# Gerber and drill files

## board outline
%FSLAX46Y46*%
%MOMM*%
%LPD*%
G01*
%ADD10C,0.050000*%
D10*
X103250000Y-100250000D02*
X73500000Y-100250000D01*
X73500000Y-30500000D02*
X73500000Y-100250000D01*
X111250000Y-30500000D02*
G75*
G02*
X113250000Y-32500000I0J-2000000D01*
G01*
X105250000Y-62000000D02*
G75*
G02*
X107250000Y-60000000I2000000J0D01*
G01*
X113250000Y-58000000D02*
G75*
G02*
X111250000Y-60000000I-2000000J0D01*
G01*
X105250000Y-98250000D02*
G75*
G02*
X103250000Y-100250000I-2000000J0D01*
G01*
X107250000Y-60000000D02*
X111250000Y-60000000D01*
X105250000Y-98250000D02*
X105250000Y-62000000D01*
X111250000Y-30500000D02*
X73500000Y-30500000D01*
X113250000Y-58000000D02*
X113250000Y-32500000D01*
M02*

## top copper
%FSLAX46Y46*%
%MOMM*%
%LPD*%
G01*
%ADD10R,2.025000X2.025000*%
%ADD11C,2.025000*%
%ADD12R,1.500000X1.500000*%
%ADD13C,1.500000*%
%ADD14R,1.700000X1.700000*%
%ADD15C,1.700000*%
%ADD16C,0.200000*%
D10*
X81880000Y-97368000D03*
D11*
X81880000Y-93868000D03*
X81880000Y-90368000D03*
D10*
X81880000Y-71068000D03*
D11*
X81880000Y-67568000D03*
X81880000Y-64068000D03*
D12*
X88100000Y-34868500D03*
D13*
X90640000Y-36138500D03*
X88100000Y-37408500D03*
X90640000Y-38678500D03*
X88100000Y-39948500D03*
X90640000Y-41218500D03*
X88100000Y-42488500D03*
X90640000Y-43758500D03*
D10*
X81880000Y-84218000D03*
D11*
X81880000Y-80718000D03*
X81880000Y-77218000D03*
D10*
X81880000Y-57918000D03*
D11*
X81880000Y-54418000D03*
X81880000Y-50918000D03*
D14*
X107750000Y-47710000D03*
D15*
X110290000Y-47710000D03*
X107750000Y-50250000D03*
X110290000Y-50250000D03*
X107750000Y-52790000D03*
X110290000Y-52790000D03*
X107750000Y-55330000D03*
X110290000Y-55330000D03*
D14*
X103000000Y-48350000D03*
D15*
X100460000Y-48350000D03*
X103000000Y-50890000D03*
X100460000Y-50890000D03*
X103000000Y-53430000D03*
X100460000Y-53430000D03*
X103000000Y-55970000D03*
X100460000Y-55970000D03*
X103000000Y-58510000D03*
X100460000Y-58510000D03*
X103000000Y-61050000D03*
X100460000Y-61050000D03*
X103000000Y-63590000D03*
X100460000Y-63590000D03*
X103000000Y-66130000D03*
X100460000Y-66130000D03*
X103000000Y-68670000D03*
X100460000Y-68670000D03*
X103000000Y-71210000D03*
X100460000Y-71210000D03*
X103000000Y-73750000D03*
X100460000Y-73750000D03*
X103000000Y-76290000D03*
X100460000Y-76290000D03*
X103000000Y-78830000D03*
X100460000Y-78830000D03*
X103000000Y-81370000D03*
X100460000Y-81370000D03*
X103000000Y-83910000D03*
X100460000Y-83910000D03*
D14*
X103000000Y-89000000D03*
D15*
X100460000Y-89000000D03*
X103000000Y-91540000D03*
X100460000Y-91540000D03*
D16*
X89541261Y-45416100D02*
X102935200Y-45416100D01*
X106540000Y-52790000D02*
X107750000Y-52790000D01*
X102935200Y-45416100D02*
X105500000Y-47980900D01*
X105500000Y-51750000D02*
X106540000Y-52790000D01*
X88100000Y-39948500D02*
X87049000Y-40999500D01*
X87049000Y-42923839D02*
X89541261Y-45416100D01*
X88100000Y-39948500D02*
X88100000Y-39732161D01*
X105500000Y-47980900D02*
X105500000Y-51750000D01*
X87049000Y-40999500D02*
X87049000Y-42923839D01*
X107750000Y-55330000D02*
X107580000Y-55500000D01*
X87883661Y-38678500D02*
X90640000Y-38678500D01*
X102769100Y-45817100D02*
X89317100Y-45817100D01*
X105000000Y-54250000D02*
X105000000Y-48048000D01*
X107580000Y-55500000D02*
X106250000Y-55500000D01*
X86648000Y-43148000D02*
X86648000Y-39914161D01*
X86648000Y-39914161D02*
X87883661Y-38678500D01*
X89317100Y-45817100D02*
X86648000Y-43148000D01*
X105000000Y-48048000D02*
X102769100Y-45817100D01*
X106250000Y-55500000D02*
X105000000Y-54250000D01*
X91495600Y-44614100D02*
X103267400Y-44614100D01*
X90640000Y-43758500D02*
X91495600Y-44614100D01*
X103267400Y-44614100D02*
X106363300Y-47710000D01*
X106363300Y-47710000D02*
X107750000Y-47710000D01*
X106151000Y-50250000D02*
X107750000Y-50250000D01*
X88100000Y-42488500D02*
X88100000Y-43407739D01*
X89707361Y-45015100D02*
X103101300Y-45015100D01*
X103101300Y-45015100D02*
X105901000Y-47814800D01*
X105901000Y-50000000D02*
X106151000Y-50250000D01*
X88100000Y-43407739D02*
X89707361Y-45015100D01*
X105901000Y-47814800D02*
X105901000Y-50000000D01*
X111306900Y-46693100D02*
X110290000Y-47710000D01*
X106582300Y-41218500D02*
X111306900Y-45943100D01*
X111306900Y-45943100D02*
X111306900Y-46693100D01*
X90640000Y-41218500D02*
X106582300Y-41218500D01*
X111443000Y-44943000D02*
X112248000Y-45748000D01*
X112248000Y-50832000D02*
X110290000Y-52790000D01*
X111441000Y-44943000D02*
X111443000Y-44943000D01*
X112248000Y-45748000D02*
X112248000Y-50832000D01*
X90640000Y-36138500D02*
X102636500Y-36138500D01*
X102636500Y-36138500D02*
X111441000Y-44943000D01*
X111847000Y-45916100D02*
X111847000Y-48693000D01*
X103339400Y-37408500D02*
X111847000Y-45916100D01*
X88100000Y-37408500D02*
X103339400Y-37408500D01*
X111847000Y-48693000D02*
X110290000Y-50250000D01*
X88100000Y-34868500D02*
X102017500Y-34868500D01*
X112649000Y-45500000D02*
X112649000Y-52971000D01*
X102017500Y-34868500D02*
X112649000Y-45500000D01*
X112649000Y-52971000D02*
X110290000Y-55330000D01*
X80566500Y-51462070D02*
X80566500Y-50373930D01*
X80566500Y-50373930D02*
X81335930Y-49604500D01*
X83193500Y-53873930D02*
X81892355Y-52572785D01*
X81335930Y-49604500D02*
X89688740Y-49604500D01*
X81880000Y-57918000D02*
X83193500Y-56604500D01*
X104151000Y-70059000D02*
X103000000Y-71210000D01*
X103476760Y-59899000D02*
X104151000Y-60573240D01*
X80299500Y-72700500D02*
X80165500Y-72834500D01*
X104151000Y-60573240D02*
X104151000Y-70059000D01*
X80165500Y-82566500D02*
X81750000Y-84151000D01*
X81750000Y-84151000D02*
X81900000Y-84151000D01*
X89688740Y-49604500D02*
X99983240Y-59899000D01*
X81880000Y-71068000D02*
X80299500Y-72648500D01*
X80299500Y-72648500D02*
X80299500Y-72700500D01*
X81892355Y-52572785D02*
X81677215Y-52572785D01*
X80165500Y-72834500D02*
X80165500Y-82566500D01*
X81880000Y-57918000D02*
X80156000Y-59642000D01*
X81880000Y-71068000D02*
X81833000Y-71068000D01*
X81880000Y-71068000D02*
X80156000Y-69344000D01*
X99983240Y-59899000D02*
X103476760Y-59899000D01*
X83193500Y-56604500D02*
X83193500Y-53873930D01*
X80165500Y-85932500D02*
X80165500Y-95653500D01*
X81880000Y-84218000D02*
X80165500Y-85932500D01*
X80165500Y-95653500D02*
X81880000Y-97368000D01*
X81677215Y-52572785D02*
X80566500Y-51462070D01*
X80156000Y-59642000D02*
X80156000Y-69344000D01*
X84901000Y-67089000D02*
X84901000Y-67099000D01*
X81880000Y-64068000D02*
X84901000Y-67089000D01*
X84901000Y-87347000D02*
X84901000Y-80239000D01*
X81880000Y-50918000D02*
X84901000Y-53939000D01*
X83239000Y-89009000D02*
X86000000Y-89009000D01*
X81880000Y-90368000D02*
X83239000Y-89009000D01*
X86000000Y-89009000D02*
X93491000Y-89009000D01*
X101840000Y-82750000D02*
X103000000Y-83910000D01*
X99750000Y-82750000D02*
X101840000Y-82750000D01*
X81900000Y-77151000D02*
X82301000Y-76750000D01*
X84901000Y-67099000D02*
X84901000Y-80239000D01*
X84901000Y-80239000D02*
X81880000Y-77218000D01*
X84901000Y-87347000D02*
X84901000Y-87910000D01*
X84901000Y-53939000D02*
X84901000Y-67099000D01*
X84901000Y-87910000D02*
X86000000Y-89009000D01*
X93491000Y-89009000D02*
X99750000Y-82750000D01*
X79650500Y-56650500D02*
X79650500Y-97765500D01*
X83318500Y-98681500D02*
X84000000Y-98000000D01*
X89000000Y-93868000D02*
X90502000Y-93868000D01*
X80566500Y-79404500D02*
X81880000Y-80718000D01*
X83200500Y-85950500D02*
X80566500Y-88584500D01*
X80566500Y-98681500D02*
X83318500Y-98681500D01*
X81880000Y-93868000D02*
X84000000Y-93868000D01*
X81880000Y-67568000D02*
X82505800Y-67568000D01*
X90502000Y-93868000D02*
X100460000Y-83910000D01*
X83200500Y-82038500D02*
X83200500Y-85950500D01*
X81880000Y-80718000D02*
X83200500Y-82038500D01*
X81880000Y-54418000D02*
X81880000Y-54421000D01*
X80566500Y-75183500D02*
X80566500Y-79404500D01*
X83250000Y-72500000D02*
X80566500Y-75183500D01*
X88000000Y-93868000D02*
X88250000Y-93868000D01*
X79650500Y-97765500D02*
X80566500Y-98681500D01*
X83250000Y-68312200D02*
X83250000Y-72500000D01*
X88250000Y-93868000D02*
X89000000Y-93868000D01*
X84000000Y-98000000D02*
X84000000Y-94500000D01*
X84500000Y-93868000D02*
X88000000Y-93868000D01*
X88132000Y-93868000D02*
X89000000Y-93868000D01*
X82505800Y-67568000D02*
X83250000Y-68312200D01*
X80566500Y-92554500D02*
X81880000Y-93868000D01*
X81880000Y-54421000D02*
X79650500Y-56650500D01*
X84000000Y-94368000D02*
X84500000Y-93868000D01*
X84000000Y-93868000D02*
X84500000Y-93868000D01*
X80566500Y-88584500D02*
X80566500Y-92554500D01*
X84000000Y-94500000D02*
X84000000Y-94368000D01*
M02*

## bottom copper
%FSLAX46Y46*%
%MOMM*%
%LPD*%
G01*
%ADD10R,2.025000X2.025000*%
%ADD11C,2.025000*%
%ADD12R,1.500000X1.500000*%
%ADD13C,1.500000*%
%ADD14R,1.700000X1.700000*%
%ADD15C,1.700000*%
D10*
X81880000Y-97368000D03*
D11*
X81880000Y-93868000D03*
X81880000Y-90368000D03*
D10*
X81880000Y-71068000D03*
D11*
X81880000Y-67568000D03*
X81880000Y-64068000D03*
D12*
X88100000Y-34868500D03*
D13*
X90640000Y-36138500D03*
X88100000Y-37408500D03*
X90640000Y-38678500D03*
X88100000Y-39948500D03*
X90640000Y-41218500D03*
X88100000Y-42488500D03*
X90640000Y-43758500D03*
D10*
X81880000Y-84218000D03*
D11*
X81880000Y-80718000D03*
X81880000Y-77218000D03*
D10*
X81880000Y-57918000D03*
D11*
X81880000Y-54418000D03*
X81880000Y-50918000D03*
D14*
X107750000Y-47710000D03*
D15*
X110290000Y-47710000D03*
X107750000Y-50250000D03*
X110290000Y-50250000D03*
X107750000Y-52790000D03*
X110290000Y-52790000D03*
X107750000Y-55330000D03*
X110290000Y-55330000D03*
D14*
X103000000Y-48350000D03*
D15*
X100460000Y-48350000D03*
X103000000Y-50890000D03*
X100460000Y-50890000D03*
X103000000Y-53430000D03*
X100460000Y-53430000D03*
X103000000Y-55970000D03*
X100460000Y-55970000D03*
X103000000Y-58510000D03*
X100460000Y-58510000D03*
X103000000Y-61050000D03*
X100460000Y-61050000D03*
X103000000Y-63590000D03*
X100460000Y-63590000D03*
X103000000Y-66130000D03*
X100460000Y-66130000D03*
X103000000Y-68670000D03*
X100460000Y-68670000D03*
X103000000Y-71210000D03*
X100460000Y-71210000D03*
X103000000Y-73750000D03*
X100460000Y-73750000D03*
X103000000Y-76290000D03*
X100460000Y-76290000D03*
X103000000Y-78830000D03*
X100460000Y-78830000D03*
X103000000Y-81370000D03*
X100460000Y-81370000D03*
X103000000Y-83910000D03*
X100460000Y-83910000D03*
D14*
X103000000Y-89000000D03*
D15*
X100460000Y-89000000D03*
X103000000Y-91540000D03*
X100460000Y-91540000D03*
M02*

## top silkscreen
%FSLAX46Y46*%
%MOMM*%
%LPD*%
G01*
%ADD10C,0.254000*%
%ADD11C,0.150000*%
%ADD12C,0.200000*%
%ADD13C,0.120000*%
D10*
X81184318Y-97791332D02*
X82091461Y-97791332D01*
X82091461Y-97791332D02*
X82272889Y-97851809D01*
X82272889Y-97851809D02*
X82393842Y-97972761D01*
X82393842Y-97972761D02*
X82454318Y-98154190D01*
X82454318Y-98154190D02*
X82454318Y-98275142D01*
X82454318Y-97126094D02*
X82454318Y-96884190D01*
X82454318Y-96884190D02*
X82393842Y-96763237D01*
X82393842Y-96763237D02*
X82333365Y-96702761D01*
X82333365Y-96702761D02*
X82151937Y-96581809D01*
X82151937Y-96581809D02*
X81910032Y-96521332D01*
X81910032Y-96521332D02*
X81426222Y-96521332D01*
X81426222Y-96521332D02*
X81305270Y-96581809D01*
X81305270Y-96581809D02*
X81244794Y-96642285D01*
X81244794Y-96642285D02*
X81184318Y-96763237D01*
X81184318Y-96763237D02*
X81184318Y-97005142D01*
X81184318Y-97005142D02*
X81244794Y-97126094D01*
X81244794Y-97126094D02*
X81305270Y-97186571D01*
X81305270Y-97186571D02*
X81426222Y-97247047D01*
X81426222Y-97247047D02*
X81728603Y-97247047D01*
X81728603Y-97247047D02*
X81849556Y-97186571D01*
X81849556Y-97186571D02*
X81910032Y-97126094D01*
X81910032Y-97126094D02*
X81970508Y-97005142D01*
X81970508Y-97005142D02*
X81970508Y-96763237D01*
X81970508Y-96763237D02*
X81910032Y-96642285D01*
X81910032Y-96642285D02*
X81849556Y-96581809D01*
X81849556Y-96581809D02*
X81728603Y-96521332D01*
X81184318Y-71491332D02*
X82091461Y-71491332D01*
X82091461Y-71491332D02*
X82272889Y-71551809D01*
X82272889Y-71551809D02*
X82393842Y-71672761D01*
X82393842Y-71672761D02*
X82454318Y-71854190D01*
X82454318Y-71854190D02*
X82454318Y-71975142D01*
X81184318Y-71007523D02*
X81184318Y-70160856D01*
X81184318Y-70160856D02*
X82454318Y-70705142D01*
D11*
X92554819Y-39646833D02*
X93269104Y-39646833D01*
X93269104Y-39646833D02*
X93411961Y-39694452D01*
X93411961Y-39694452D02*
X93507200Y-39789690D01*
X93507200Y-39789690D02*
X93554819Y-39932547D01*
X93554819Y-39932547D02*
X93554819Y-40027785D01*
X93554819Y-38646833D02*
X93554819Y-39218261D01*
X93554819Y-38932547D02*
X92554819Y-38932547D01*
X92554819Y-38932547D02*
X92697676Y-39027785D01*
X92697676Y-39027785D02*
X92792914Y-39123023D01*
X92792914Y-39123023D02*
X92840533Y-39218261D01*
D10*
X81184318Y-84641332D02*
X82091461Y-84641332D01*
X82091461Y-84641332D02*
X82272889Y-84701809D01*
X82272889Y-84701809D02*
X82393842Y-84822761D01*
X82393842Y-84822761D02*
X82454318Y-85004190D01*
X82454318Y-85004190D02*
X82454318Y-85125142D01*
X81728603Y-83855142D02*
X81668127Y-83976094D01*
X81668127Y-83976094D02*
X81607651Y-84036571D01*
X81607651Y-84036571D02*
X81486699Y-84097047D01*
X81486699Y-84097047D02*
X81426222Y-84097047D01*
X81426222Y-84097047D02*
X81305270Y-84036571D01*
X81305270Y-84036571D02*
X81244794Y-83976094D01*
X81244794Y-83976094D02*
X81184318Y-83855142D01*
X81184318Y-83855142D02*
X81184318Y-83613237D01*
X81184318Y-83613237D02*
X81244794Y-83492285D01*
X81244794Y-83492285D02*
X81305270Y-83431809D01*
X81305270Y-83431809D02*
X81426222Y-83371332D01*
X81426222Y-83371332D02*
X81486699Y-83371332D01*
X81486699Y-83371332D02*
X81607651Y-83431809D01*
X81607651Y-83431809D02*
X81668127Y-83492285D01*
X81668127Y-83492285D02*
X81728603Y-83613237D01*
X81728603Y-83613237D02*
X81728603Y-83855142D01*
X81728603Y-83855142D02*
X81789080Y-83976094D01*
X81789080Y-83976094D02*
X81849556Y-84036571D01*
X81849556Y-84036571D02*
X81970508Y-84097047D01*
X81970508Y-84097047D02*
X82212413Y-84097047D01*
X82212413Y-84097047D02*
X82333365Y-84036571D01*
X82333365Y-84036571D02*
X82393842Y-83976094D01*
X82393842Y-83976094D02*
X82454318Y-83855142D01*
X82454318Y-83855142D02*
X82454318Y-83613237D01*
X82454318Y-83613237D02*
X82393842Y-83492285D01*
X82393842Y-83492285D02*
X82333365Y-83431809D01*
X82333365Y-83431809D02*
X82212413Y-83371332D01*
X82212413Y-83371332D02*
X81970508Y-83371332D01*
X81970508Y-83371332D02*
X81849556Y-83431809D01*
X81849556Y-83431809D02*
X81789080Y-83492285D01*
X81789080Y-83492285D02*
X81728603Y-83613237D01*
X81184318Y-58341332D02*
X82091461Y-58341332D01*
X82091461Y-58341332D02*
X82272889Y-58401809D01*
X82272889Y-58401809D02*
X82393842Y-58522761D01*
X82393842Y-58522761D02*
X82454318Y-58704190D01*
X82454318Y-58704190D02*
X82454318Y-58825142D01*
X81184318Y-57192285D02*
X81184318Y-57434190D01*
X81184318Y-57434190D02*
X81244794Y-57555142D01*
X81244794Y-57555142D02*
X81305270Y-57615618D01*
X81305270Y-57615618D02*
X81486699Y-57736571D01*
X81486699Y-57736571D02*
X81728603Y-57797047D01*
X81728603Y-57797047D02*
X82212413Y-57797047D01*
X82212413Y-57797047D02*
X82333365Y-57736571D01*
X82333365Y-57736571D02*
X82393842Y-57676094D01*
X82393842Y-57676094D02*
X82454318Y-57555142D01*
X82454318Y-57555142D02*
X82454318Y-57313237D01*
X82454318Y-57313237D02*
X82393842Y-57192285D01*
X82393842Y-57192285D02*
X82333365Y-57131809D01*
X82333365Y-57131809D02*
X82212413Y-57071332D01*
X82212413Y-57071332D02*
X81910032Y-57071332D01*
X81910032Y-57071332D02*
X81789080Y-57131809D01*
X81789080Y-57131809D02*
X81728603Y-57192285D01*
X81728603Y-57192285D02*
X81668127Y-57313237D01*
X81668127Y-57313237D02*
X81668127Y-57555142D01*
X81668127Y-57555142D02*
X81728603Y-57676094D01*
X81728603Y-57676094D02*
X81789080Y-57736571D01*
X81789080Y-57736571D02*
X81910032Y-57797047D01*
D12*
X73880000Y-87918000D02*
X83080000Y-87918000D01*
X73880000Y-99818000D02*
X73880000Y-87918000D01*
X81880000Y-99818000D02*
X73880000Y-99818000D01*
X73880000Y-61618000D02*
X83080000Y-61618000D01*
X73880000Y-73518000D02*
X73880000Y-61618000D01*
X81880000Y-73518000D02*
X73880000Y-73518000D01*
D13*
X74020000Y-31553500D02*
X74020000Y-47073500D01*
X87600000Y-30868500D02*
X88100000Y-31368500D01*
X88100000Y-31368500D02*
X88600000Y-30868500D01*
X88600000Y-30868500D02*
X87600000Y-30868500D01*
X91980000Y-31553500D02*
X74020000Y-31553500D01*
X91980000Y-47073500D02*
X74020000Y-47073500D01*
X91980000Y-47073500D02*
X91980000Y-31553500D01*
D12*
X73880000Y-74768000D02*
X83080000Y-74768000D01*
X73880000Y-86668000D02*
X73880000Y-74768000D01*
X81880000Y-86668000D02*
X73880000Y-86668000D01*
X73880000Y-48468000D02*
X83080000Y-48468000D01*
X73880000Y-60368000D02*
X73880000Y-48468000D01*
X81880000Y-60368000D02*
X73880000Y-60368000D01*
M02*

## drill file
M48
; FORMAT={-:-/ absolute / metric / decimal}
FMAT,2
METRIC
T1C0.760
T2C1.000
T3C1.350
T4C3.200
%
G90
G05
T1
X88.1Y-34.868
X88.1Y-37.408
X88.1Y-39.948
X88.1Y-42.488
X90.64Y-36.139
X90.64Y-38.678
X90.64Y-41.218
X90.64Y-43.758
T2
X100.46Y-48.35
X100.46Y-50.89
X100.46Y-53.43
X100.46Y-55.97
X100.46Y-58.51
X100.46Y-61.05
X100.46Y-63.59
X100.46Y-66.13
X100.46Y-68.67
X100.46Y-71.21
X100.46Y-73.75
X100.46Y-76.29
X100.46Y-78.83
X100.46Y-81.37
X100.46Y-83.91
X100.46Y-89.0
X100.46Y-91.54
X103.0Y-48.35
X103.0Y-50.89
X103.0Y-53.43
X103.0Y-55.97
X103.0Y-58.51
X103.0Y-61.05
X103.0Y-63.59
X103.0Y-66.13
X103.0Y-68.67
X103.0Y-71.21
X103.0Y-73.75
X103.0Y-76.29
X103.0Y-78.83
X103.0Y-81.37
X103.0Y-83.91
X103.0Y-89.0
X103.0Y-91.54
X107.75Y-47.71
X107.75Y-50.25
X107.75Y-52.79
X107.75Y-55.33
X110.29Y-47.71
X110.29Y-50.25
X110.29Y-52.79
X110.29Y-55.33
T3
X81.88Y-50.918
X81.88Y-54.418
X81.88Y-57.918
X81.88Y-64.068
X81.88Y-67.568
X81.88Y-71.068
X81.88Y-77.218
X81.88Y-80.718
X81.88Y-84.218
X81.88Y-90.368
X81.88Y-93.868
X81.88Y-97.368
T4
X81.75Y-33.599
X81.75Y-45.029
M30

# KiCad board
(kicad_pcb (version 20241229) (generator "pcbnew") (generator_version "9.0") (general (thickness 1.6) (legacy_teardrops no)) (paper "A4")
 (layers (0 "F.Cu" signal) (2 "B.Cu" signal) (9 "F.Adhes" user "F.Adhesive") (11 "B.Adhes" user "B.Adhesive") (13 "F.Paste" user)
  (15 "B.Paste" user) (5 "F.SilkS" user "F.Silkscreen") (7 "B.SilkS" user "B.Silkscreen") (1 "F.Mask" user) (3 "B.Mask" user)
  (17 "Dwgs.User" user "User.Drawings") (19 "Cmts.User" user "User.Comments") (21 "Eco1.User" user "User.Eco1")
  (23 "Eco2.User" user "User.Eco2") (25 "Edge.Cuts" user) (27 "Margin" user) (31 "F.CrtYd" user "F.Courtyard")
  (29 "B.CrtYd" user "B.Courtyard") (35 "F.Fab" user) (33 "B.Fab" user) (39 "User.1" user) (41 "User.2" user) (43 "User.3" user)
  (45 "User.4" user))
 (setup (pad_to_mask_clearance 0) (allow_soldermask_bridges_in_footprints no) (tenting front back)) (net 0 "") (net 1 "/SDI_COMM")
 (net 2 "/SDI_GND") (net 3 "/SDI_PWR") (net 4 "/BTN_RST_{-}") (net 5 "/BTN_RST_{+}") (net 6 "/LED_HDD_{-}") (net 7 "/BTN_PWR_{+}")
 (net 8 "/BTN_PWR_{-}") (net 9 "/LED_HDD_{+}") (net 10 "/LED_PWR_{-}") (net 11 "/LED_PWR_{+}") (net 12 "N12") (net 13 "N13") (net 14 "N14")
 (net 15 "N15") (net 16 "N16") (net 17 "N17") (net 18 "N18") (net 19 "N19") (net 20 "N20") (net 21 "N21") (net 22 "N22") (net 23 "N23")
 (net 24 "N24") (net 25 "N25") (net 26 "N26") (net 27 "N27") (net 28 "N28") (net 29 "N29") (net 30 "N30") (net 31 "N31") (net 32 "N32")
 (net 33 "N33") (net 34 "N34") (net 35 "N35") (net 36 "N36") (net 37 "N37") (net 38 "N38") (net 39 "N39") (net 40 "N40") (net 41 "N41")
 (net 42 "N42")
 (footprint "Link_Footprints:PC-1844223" (layer "F.Cu") (at 81.88 97.368 90)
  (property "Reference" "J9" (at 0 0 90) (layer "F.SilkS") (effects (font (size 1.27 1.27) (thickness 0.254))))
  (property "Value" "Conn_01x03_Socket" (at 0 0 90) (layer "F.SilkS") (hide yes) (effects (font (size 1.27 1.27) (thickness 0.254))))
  (fp_line (start 9.45 -8) (end 9.45 1.2) (stroke (width 0.2) (type solid)) (layer "F.SilkS"))
  (fp_line (start -2.45 -8) (end 9.45 -8) (stroke (width 0.2) (type solid)) (layer "F.SilkS"))
  (fp_line (start -2.45 0) (end -2.45 -8) (stroke (width 0.2) (type solid)) (layer "F.SilkS"))
  (pad "1" thru_hole rect (at 0 0 90) (size 2.025 2.025) (drill 1.35) (layers "*.Cu" "*.Mask") (remove_unused_layers no) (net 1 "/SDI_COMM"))
  (pad "2" thru_hole circle (at 3.5 0 90) (size 2.025 2.025) (drill 1.35) (layers "*.Cu" "*.Mask") (remove_unused_layers no)
   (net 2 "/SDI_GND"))
  (pad "3" thru_hole circle (at 7 0 90) (size 2.025 2.025) (drill 1.35) (layers "*.Cu" "*.Mask") (remove_unused_layers no)
   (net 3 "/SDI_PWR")))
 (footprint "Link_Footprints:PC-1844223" (layer "F.Cu") (at 81.88 71.068 90)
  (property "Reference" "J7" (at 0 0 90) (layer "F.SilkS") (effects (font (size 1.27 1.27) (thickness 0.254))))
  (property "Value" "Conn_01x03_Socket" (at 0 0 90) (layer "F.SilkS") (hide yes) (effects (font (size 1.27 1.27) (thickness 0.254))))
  (fp_line (start 9.45 -8) (end 9.45 1.2) (stroke (width 0.2) (type solid)) (layer "F.SilkS"))
  (fp_line (start -2.45 -8) (end 9.45 -8) (stroke (width 0.2) (type solid)) (layer "F.SilkS"))
  (fp_line (start -2.45 0) (end -2.45 -8) (stroke (width 0.2) (type solid)) (layer "F.SilkS"))
  (pad "1" thru_hole rect (at 0 0 90) (size 2.025 2.025) (drill 1.35) (layers "*.Cu" "*.Mask") (remove_unused_layers no) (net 1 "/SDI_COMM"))
  (pad "2" thru_hole circle (at 3.5 0 90) (size 2.025 2.025) (drill 1.35) (layers "*.Cu" "*.Mask") (remove_unused_layers no)
   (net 2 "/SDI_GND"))
  (pad "3" thru_hole circle (at 7 0 90) (size 2.025 2.025) (drill 1.35) (layers "*.Cu" "*.Mask") (remove_unused_layers no)
   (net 3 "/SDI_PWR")))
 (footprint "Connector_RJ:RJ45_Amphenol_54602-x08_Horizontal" (layer "F.Cu") (at 88.1 34.8685 -90)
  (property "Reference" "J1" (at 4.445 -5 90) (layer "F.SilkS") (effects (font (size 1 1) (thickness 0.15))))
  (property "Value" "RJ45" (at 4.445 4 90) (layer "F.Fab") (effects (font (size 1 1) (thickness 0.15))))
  (fp_line (start -3.315 14.08) (end 12.205 14.08) (stroke (width 0.12) (type solid)) (layer "F.SilkS"))
  (fp_line (start -4 0.5) (end -3.5 0) (stroke (width 0.12) (type solid)) (layer "F.SilkS"))
  (fp_line (start -3.5 0) (end -4 -0.5) (stroke (width 0.12) (type solid)) (layer "F.SilkS"))
  (fp_line (start -4 -0.5) (end -4 0.5) (stroke (width 0.12) (type solid)) (layer "F.SilkS"))
  (fp_line (start -3.315 -3.88) (end -3.315 14.08) (stroke (width 0.12) (type solid)) (layer "F.SilkS"))
  (fp_line (start 12.205 -3.88) (end 12.205 14.08) (stroke (width 0.12) (type solid)) (layer "F.SilkS"))
  (fp_line (start 12.205 -3.88) (end -3.315 -3.88) (stroke (width 0.12) (type solid)) (layer "F.SilkS"))
  (pad "" np_thru_hole circle (at -1.27 6.35 270) (size 3.2 3.2) (drill 3.2) (layers "*.Cu" "*.Mask"))
  (pad "" np_thru_hole circle (at 10.16 6.35 270) (size 3.2 3.2) (drill 3.2) (layers "*.Cu" "*.Mask"))
  (pad "1" thru_hole rect (at 0 0 270) (size 1.5 1.5) (drill 0.76) (layers "*.Cu" "*.Mask") (remove_unused_layers no) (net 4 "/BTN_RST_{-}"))
  (pad "2" thru_hole circle (at 1.27 -2.54 270) (size 1.5 1.5) (drill 0.76) (layers "*.Cu" "*.Mask") (remove_unused_layers no)
   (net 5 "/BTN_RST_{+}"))
  (pad "3" thru_hole circle (at 2.54 0 270) (size 1.5 1.5) (drill 0.76) (layers "*.Cu" "*.Mask") (remove_unused_layers no)
   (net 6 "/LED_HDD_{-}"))
  (pad "4" thru_hole circle (at 3.81 -2.54 270) (size 1.5 1.5) (drill 0.76) (layers "*.Cu" "*.Mask") (remove_unused_layers no)
   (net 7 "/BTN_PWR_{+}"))
  (pad "5" thru_hole circle (at 5.08 0 270) (size 1.5 1.5) (drill 0.76) (layers "*.Cu" "*.Mask") (remove_unused_layers no)
   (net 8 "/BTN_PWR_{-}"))
  (pad "6" thru_hole circle (at 6.35 -2.54 270) (size 1.5 1.5) (drill 0.76) (layers "*.Cu" "*.Mask") (remove_unused_layers no)
   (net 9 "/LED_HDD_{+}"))
  (pad "7" thru_hole circle (at 7.62 0 270) (size 1.5 1.5) (drill 0.76) (layers "*.Cu" "*.Mask") (remove_unused_layers no)
   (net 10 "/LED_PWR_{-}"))
  (pad "8" thru_hole circle (at 8.89 -2.54 270) (size 1.5 1.5) (drill 0.76) (layers "*.Cu" "*.Mask") (remove_unused_layers no)
   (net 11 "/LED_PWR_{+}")))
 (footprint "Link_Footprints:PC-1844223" (layer "F.Cu") (at 81.88 84.218 90)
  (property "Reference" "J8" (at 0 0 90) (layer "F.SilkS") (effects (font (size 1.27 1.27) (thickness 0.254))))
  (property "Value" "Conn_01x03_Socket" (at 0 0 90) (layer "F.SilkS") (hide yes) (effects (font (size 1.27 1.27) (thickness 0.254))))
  (fp_line (start 9.45 -8) (end 9.45 1.2) (stroke (width 0.2) (type solid)) (layer "F.SilkS"))
  (fp_line (start -2.45 -8) (end 9.45 -8) (stroke (width 0.2) (type solid)) (layer "F.SilkS"))
  (fp_line (start -2.45 0) (end -2.45 -8) (stroke (width 0.2) (type solid)) (layer "F.SilkS"))
  (pad "1" thru_hole rect (at 0 0 90) (size 2.025 2.025) (drill 1.35) (layers "*.Cu" "*.Mask") (remove_unused_layers no) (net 1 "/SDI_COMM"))
  (pad "2" thru_hole circle (at 3.5 0 90) (size 2.025 2.025) (drill 1.35) (layers "*.Cu" "*.Mask") (remove_unused_layers no)
   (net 2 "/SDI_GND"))
  (pad "3" thru_hole circle (at 7 0 90) (size 2.025 2.025) (drill 1.35) (layers "*.Cu" "*.Mask") (remove_unused_layers no)
   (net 3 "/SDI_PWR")))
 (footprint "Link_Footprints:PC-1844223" (layer "F.Cu") (at 81.88 57.918 90)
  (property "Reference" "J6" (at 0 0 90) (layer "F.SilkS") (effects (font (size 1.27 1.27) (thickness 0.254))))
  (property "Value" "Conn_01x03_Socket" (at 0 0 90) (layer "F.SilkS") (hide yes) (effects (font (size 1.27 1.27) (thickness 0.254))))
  (fp_line (start 9.45 -8) (end 9.45 1.2) (stroke (width 0.2) (type solid)) (layer "F.SilkS"))
  (fp_line (start -2.45 -8) (end 9.45 -8) (stroke (width 0.2) (type solid)) (layer "F.SilkS"))
  (fp_line (start -2.45 0) (end -2.45 -8) (stroke (width 0.2) (type solid)) (layer "F.SilkS"))
  (pad "1" thru_hole rect (at 0 0 90) (size 2.025 2.025) (drill 1.35) (layers "*.Cu" "*.Mask") (remove_unused_layers no) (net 1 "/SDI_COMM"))
  (pad "2" thru_hole circle (at 3.5 0 90) (size 2.025 2.025) (drill 1.35) (layers "*.Cu" "*.Mask") (remove_unused_layers no)
   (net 2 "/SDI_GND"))
  (pad "3" thru_hole circle (at 7 0 90) (size 2.025 2.025) (drill 1.35) (layers "*.Cu" "*.Mask") (remove_unused_layers no)
   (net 3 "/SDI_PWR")))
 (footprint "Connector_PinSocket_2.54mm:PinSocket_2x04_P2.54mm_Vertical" (layer "B.Cu") (at 107.75 47.71 180)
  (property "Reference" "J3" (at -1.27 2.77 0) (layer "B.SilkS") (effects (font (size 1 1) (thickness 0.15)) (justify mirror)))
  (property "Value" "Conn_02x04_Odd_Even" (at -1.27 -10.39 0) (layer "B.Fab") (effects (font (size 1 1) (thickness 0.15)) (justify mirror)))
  (pad "1" thru_hole rect (at 0 0 180) (size 1.7 1.7) (drill 1) (layers "*.Cu" "*.Mask") (remove_unused_layers no) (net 11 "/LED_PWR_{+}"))
  (pad "2" thru_hole circle (at -2.54 0 180) (size 1.7 1.7) (drill 1) (layers "*.Cu" "*.Mask") (remove_unused_layers no)
   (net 9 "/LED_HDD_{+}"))
  (pad "3" thru_hole circle (at 0 -2.54 180) (size 1.7 1.7) (drill 1) (layers "*.Cu" "*.Mask") (remove_unused_layers no)
   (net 10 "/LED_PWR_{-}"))
  (pad "4" thru_hole circle (at -2.54 -2.54 180) (size 1.7 1.7) (drill 1) (layers "*.Cu" "*.Mask") (remove_unused_layers no)
   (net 6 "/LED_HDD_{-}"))
  (pad "5" thru_hole circle (at 0 -5.08 180) (size 1.7 1.7) (drill 1) (layers "*.Cu" "*.Mask") (remove_unused_layers no)
   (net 8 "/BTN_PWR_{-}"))
  (pad "6" thru_hole circle (at -2.54 -5.08 180) (size 1.7 1.7) (drill 1) (layers "*.Cu" "*.Mask") (remove_unused_layers no)
   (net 5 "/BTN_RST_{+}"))
  (pad "7" thru_hole circle (at 0 -7.62 180) (size 1.7 1.7) (drill 1) (layers "*.Cu" "*.Mask") (remove_unused_layers no)
   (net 7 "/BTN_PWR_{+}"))
  (pad "8" thru_hole circle (at -2.54 -7.62 180) (size 1.7 1.7) (drill 1) (layers "*.Cu" "*.Mask") (remove_unused_layers no)
   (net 4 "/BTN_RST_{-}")))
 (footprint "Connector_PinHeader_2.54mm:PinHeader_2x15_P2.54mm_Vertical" (layer "B.Cu") (at 103 48.35 180)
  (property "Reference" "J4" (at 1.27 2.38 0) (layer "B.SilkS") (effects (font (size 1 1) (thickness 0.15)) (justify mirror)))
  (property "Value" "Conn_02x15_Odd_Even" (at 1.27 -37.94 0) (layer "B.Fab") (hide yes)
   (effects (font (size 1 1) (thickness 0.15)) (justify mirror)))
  (pad "1" thru_hole rect (at 0 0 180) (size 1.7 1.7) (drill 1) (layers "*.Cu" "*.Mask") (remove_unused_layers no) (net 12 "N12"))
  (pad "2" thru_hole circle (at 2.54 0 180) (size 1.7 1.7) (drill 1) (layers "*.Cu" "*.Mask") (remove_unused_layers no) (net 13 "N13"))
  (pad "3" thru_hole circle (at 0 -2.54 180) (size 1.7 1.7) (drill 1) (layers "*.Cu" "*.Mask") (remove_unused_layers no) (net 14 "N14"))
  (pad "4" thru_hole circle (at 2.54 -2.54 180) (size 1.7 1.7) (drill 1) (layers "*.Cu" "*.Mask") (remove_unused_layers no) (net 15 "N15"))
  (pad "5" thru_hole circle (at 0 -5.08 180) (size 1.7 1.7) (drill 1) (layers "*.Cu" "*.Mask") (remove_unused_layers no) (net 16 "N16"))
  (pad "6" thru_hole circle (at 2.54 -5.08 180) (size 1.7 1.7) (drill 1) (layers "*.Cu" "*.Mask") (remove_unused_layers no) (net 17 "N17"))
  (pad "7" thru_hole circle (at 0 -7.62 180) (size 1.7 1.7) (drill 1) (layers "*.Cu" "*.Mask") (remove_unused_layers no) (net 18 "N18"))
  (pad "8" thru_hole circle (at 2.54 -7.62 180) (size 1.7 1.7) (drill 1) (layers "*.Cu" "*.Mask") (remove_unused_layers no) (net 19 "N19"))
  (pad "9" thru_hole circle (at 0 -10.16 180) (size 1.7 1.7) (drill 1) (layers "*.Cu" "*.Mask") (remove_unused_layers no) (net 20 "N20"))
  (pad "10" thru_hole circle (at 2.54 -10.16 180) (size 1.7 1.7) (drill 1) (layers "*.Cu" "*.Mask") (remove_unused_layers no) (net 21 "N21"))
  (pad "11" thru_hole circle (at 0 -12.7 180) (size 1.7 1.7) (drill 1) (layers "*.Cu" "*.Mask") (remove_unused_layers no) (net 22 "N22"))
  (pad "12" thru_hole circle (at 2.54 -12.7 180) (size 1.7 1.7) (drill 1) (layers "*.Cu" "*.Mask") (remove_unused_layers no) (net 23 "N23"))
  (pad "13" thru_hole circle (at 0 -15.24 180) (size 1.7 1.7) (drill 1) (layers "*.Cu" "*.Mask") (remove_unused_layers no) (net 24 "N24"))
  (pad "14" thru_hole circle (at 2.54 -15.24 180) (size 1.7 1.7) (drill 1) (layers "*.Cu" "*.Mask") (remove_unused_layers no) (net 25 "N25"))
  (pad "15" thru_hole circle (at 0 -17.78 180) (size 1.7 1.7) (drill 1) (layers "*.Cu" "*.Mask") (remove_unused_layers no) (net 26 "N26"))
  (pad "16" thru_hole circle (at 2.54 -17.78 180) (size 1.7 1.7) (drill 1) (layers "*.Cu" "*.Mask") (remove_unused_layers no) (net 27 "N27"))
  (pad "17" thru_hole circle (at 0 -20.32 180) (size 1.7 1.7) (drill 1) (layers "*.Cu" "*.Mask") (remove_unused_layers no) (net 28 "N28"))
  (pad "18" thru_hole circle (at 2.54 -20.32 180) (size 1.7 1.7) (drill 1) (layers "*.Cu" "*.Mask") (remove_unused_layers no) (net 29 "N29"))
  (pad "19" thru_hole circle (at 0 -22.86 180) (size 1.7 1.7) (drill 1) (layers "*.Cu" "*.Mask") (remove_unused_layers no)
   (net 1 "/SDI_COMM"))
  (pad "20" thru_hole circle (at 2.54 -22.86 180) (size 1.7 1.7) (drill 1) (layers "*.Cu" "*.Mask") (remove_unused_layers no) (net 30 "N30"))
  (pad "21" thru_hole circle (at 0 -25.4 180) (size 1.7 1.7) (drill 1) (layers "*.Cu" "*.Mask") (remove_unused_layers no) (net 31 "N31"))
  (pad "22" thru_hole circle (at 2.54 -25.4 180) (size 1.7 1.7) (drill 1) (layers "*.Cu" "*.Mask") (remove_unused_layers no) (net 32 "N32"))
  (pad "23" thru_hole circle (at 0 -27.94 180) (size 1.7 1.7) (drill 1) (layers "*.Cu" "*.Mask") (remove_unused_layers no) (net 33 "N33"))
  (pad "24" thru_hole circle (at 2.54 -27.94 180) (size 1.7 1.7) (drill 1) (layers "*.Cu" "*.Mask") (remove_unused_layers no) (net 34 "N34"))
  (pad "25" thru_hole circle (at 0 -30.48 180) (size 1.7 1.7) (drill 1) (layers "*.Cu" "*.Mask") (remove_unused_layers no) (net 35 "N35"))
  (pad "26" thru_hole circle (at 2.54 -30.48 180) (size 1.7 1.7) (drill 1) (layers "*.Cu" "*.Mask") (remove_unused_layers no) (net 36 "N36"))
  (pad "27" thru_hole circle (at 0 -33.02 180) (size 1.7 1.7) (drill 1) (layers "*.Cu" "*.Mask") (remove_unused_layers no) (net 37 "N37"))
  (pad "28" thru_hole circle (at 2.54 -33.02 180) (size 1.7 1.7) (drill 1) (layers "*.Cu" "*.Mask") (remove_unused_layers no) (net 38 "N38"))
  (pad "29" thru_hole circle (at 0 -35.56 180) (size 1.7 1.7) (drill 1) (layers "*.Cu" "*.Mask") (remove_unused_layers no)
   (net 3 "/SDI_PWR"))
  (pad "30" thru_hole circle (at 2.54 -35.56 180) (size 1.7 1.7) (drill 1) (layers "*.Cu" "*.Mask") (remove_unused_layers no)
   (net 2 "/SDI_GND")))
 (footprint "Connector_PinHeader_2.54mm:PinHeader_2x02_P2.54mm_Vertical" (layer "B.Cu") (at 103 89 180)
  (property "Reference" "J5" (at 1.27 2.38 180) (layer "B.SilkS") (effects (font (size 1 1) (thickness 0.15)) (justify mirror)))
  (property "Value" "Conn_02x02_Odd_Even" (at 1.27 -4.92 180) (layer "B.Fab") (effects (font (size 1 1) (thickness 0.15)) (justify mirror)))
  (pad "1" thru_hole rect (at 0 0 180) (size 1.7 1.7) (drill 1) (layers "*.Cu" "*.Mask") (remove_unused_layers no) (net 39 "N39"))
  (pad "2" thru_hole circle (at 2.54 0 180) (size 1.7 1.7) (drill 1) (layers "*.Cu" "*.Mask") (remove_unused_layers no) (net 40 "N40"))
  (pad "3" thru_hole circle (at 0 -2.54 180) (size 1.7 1.7) (drill 1) (layers "*.Cu" "*.Mask") (remove_unused_layers no) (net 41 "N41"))
  (pad "4" thru_hole circle (at 2.54 -2.54 180) (size 1.7 1.7) (drill 1) (layers "*.Cu" "*.Mask") (remove_unused_layers no) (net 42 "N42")))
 (gr_line (start 103.25 100.25) (end 73.5 100.25) (stroke (width 0.05) (type default)) (layer "Edge.Cuts"))
 (gr_line (start 73.5 30.5) (end 73.5 100.25) (stroke (width 0.05) (type default)) (layer "Edge.Cuts"))
 (gr_arc (start 111.25 30.5) (mid 112.664214 31.085786) (end 113.25 32.5) (stroke (width 0.05) (type default)) (layer "Edge.Cuts"))
 (gr_arc (start 105.25 62) (mid 105.835786 60.585786) (end 107.25 60) (stroke (width 0.05) (type default)) (layer "Edge.Cuts"))
 (gr_arc (start 113.25 58) (mid 112.664214 59.414214) (end 111.25 60) (stroke (width 0.05) (type default)) (layer "Edge.Cuts"))
 (gr_arc (start 105.25 98.25) (mid 104.664214 99.664214) (end 103.25 100.25) (stroke (width 0.05) (type default)) (layer "Edge.Cuts"))
 (gr_line (start 107.25 60) (end 111.25 60) (stroke (width 0.05) (type default)) (layer "Edge.Cuts"))
 (gr_line (start 105.25 98.25) (end 105.25 62) (stroke (width 0.05) (type default)) (layer "Edge.Cuts"))
 (gr_line (start 111.25 30.5) (end 73.5 30.5) (stroke (width 0.05) (type default)) (layer "Edge.Cuts"))
 (gr_line (start 113.25 58) (end 113.25 32.5) (stroke (width 0.05) (type default)) (layer "Edge.Cuts"))
 (segment (start 89.541261 45.4161) (end 102.9352 45.4161) (width 0.2) (layer "F.Cu") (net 8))
 (segment (start 106.54 52.79) (end 107.75 52.79) (width 0.2) (layer "F.Cu") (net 8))
 (segment (start 102.9352 45.4161) (end 105.5 47.9809) (width 0.2) (layer "F.Cu") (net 8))
 (segment (start 105.5 51.75) (end 106.54 52.79) (width 0.2) (layer "F.Cu") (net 8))
 (segment (start 88.1 39.9485) (end 87.049 40.9995) (width 0.2) (layer "F.Cu") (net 8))
 (segment (start 87.049 42.923839) (end 89.541261 45.4161) (width 0.2) (layer "F.Cu") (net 8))
 (segment (start 88.1 39.9485) (end 88.1 39.732161) (width 0.2) (layer "F.Cu") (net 8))
 (segment (start 105.5 47.9809) (end 105.5 51.75) (width 0.2) (layer "F.Cu") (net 8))
 (segment (start 87.049 40.9995) (end 87.049 42.923839) (width 0.2) (layer "F.Cu") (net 8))
 (segment (start 107.75 55.33) (end 107.58 55.5) (width 0.2) (layer "F.Cu") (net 7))
 (segment (start 87.883661 38.6785) (end 90.64 38.6785) (width 0.2) (layer "F.Cu") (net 7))
 (segment (start 102.7691 45.8171) (end 89.3171 45.8171) (width 0.2) (layer "F.Cu") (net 7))
 (segment (start 105 54.25) (end 105 48.048) (width 0.2) (layer "F.Cu") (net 7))
 (segment (start 107.58 55.5) (end 106.25 55.5) (width 0.2) (layer "F.Cu") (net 7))
 (segment (start 86.648 43.148) (end 86.648 39.914161) (width 0.2) (layer "F.Cu") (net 7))
 (segment (start 86.648 39.914161) (end 87.883661 38.6785) (width 0.2) (layer "F.Cu") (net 7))
 (segment (start 89.3171 45.8171) (end 86.648 43.148) (width 0.2) (layer "F.Cu") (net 7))
 (segment (start 105 48.048) (end 102.7691 45.8171) (width 0.2) (layer "F.Cu") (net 7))
 (segment (start 106.25 55.5) (end 105 54.25) (width 0.2) (layer "F.Cu") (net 7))
 (segment (start 91.4956 44.6141) (end 103.2674 44.6141) (width 0.2) (layer "F.Cu") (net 11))
 (segment (start 90.64 43.7585) (end 91.4956 44.6141) (width 0.2) (layer "F.Cu") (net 11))
 (segment (start 103.2674 44.6141) (end 106.3633 47.71) (width 0.2) (layer "F.Cu") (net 11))
 (segment (start 106.3633 47.71) (end 107.75 47.71) (width 0.2) (layer "F.Cu") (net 11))
 (segment (start 106.151 50.25) (end 107.75 50.25) (width 0.2) (layer "F.Cu") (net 10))
 (segment (start 88.1 42.4885) (end 88.1 43.407739) (width 0.2) (layer "F.Cu") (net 10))
 (segment (start 89.707361 45.0151) (end 103.1013 45.0151) (width 0.2) (layer "F.Cu") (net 10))
 (segment (start 103.1013 45.0151) (end 105.901 47.8148) (width 0.2) (layer "F.Cu") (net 10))
 (segment (start 105.901 50) (end 106.151 50.25) (width 0.2) (layer "F.Cu") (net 10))
 (segment (start 88.1 43.407739) (end 89.707361 45.0151) (width 0.2) (layer "F.Cu") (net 10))
 (segment (start 105.901 47.8148) (end 105.901 50) (width 0.2) (layer "F.Cu") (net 10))
 (segment (start 111.3069 46.6931) (end 110.29 47.71) (width 0.2) (layer "F.Cu") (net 9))
 (segment (start 106.5823 41.2185) (end 111.3069 45.9431) (width 0.2) (layer "F.Cu") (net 9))
 (segment (start 111.3069 45.9431) (end 111.3069 46.6931) (width 0.2) (layer "F.Cu") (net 9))
 (segment (start 90.64 41.2185) (end 106.5823 41.2185) (width 0.2) (layer "F.Cu") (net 9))
 (segment (start 111.443 44.943) (end 112.248 45.748) (width 0.2) (layer "F.Cu") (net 5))
 (segment (start 112.248 50.832) (end 110.29 52.79) (width 0.2) (layer "F.Cu") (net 5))
 (segment (start 111.441 44.943) (end 111.443 44.943) (width 0.2) (layer "F.Cu") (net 5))
 (segment (start 112.248 45.748) (end 112.248 50.832) (width 0.2) (layer "F.Cu") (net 5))
 (segment (start 90.64 36.1385) (end 102.6365 36.1385) (width 0.2) (layer "F.Cu") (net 5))
 (segment (start 102.6365 36.1385) (end 111.441 44.943) (width 0.2) (layer "F.Cu") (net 5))
 (segment (start 111.847 45.9161) (end 111.847 48.693) (width 0.2) (layer "F.Cu") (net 6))
 (segment (start 103.3394 37.4085) (end 111.847 45.9161) (width 0.2) (layer "F.Cu") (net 6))
 (segment (start 88.1 37.4085) (end 103.3394 37.4085) (width 0.2) (layer "F.Cu") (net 6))
 (segment (start 111.847 48.693) (end 110.29 50.25) (width 0.2) (layer "F.Cu") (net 6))
 (segment (start 88.1 34.8685) (end 102.0175 34.8685) (width 0.2) (layer "F.Cu") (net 4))
 (segment (start 112.649 45.5) (end 112.649 52.971) (width 0.2) (layer "F.Cu") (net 4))
 (segment (start 102.0175 34.8685) (end 112.649 45.5) (width 0.2) (layer "F.Cu") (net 4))
 (segment (start 112.649 52.971) (end 110.29 55.33) (width 0.2) (layer "F.Cu") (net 4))
 (segment (start 80.5665 51.46207) (end 80.5665 50.37393) (width 0.2) (layer "F.Cu") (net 1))
 (segment (start 80.5665 50.37393) (end 81.33593 49.6045) (width 0.2) (layer "F.Cu") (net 1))
 (segment (start 83.1935 53.87393) (end 81.892355 52.572785) (width 0.2) (layer "F.Cu") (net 1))
 (segment (start 81.33593 49.6045) (end 89.68874 49.6045) (width 0.2) (layer "F.Cu") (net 1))
 (segment (start 81.88 57.918) (end 83.1935 56.6045) (width 0.2) (layer "F.Cu") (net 1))
 (segment (start 104.151 70.059) (end 103 71.21) (width 0.2) (layer "F.Cu") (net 1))
 (segment (start 103.47676 59.899) (end 104.151 60.57324) (width 0.2) (layer "F.Cu") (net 1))
 (segment (start 80.2995 72.7005) (end 80.1655 72.8345) (width 0.2) (layer "F.Cu") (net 1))
 (segment (start 104.151 60.57324) (end 104.151 70.059) (width 0.2) (layer "F.Cu") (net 1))
 (segment (start 80.1655 82.5665) (end 81.75 84.151) (width 0.2) (layer "F.Cu") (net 1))
 (segment (start 81.75 84.151) (end 81.9 84.151) (width 0.2) (layer "F.Cu") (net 1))
 (segment (start 89.68874 49.6045) (end 99.98324 59.899) (width 0.2) (layer "F.Cu") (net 1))
 (segment (start 81.88 71.068) (end 80.2995 72.6485) (width 0.2) (layer "F.Cu") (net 1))
 (segment (start 80.2995 72.6485) (end 80.2995 72.7005) (width 0.2) (layer "F.Cu") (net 1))
 (segment (start 81.892355 52.572785) (end 81.677215 52.572785) (width 0.2) (layer "F.Cu") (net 1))
 (segment (start 80.1655 72.8345) (end 80.1655 82.5665) (width 0.2) (layer "F.Cu") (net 1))
 (segment (start 81.88 57.918) (end 80.156 59.642) (width 0.2) (layer "F.Cu") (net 1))
 (segment (start 81.88 71.068) (end 81.833 71.068) (width 0.2) (layer "F.Cu") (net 1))
 (segment (start 81.88 71.068) (end 80.156 69.344) (width 0.2) (layer "F.Cu") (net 1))
 (segment (start 99.98324 59.899) (end 103.47676 59.899) (width 0.2) (layer "F.Cu") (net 1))
 (segment (start 83.1935 56.6045) (end 83.1935 53.87393) (width 0.2) (layer "F.Cu") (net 1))
 (segment (start 80.1655 85.9325) (end 80.1655 95.6535) (width 0.2) (layer "F.Cu") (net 1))
 (segment (start 81.88 84.218) (end 80.1655 85.9325) (width 0.2) (layer "F.Cu") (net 1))
 (segment (start 80.1655 95.6535) (end 81.88 97.368) (width 0.2) (layer "F.Cu") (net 1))
 (segment (start 81.677215 52.572785) (end 80.5665 51.46207) (width 0.2) (layer "F.Cu") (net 1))
 (segment (start 80.156 59.642) (end 80.156 69.344) (width 0.2) (layer "F.Cu") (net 1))
 (segment (start 84.901 67.089) (end 84.901 67.099) (width 0.2) (layer "F.Cu") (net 3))
 (segment (start 81.88 64.068) (end 84.901 67.089) (width 0.2) (layer "F.Cu") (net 3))
 (segment (start 84.901 87.347) (end 84.901 80.239) (width 0.2) (layer "F.Cu") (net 3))
 (segment (start 81.88 50.918) (end 84.901 53.939) (width 0.2) (layer "F.Cu") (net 3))
 (segment (start 83.239 89.009) (end 86 89.009) (width 0.2) (layer "F.Cu") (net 3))
 (segment (start 81.88 90.368) (end 83.239 89.009) (width 0.2) (layer "F.Cu") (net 3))
 (segment (start 86 89.009) (end 93.491 89.009) (width 0.2) (layer "F.Cu") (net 3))
 (segment (start 101.84 82.75) (end 103 83.91) (width 0.2) (layer "F.Cu") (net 3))
 (segment (start 99.75 82.75) (end 101.84 82.75) (width 0.2) (layer "F.Cu") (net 3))
 (segment (start 81.9 77.151) (end 82.301 76.75) (width 0.2) (layer "F.Cu") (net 3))
 (segment (start 84.901 67.099) (end 84.901 80.239) (width 0.2) (layer "F.Cu") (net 3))
 (segment (start 84.901 80.239) (end 81.88 77.218) (width 0.2) (layer "F.Cu") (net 3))
 (segment (start 84.901 87.347) (end 84.901 87.91) (width 0.2) (layer "F.Cu") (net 3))
 (segment (start 84.901 53.939) (end 84.901 67.099) (width 0.2) (layer "F.Cu") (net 3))
 (segment (start 84.901 87.91) (end 86 89.009) (width 0.2) (layer "F.Cu") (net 3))
 (segment (start 93.491 89.009) (end 99.75 82.75) (width 0.2) (layer "F.Cu") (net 3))
 (segment (start 79.6505 56.6505) (end 79.6505 97.7655) (width 0.2) (layer "F.Cu") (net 2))
 (segment (start 83.3185 98.6815) (end 84 98) (width 0.2) (layer "F.Cu") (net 2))
 (segment (start 89 93.868) (end 90.502 93.868) (width 0.2) (layer "F.Cu") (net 2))
 (segment (start 80.5665 79.4045) (end 81.88 80.718) (width 0.2) (layer "F.Cu") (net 2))
 (segment (start 83.2005 85.9505) (end 80.5665 88.5845) (width 0.2) (layer "F.Cu") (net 2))
 (segment (start 80.5665 98.6815) (end 83.3185 98.6815) (width 0.2) (layer "F.Cu") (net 2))
 (segment (start 81.88 93.868) (end 84 93.868) (width 0.2) (layer "F.Cu") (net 2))
 (segment (start 81.88 67.568) (end 82.5058 67.568) (width 0.2) (layer "F.Cu") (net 2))
 (segment (start 90.502 93.868) (end 100.46 83.91) (width 0.2) (layer "F.Cu") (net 2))
 (segment (start 83.2005 82.0385) (end 83.2005 85.9505) (width 0.2) (layer "F.Cu") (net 2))
 (segment (start 81.88 80.718) (end 83.2005 82.0385) (width 0.2) (layer "F.Cu") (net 2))
 (segment (start 81.88 54.418) (end 81.88 54.421) (width 0.2) (layer "F.Cu") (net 2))
 (segment (start 80.5665 75.1835) (end 80.5665 79.4045) (width 0.2) (layer "F.Cu") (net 2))
 (segment (start 83.25 72.5) (end 80.5665 75.1835) (width 0.2) (layer "F.Cu") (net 2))
 (segment (start 88 93.868) (end 88.25 93.868) (width 0.2) (layer "F.Cu") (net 2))
 (segment (start 79.6505 97.7655) (end 80.5665 98.6815) (width 0.2) (layer "F.Cu") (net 2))
 (segment (start 83.25 68.3122) (end 83.25 72.5) (width 0.2) (layer "F.Cu") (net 2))
 (segment (start 88.25 93.868) (end 89 93.868) (width 0.2) (layer "F.Cu") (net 2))
 (segment (start 84 98) (end 84 94.5) (width 0.2) (layer "F.Cu") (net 2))
 (segment (start 84.5 93.868) (end 88 93.868) (width 0.2) (layer "F.Cu") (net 2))
 (segment (start 88.132 93.868) (end 89 93.868) (width 0.2) (layer "F.Cu") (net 2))
 (segment (start 82.5058 67.568) (end 83.25 68.3122) (width 0.2) (layer "F.Cu") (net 2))
 (segment (start 80.5665 92.5545) (end 81.88 93.868) (width 0.2) (layer "F.Cu") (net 2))
 (segment (start 81.88 54.421) (end 79.6505 56.6505) (width 0.2) (layer "F.Cu") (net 2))
 (segment (start 84 94.368) (end 84.5 93.868) (width 0.2) (layer "F.Cu") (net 2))
 (segment (start 84 93.868) (end 84.5 93.868) (width 0.2) (layer "F.Cu") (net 2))
 (segment (start 80.5665 88.5845) (end 80.5665 92.5545) (width 0.2) (layer "F.Cu") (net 2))
 (segment (start 84 94.5) (end 84 94.368) (width 0.2) (layer "F.Cu") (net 2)))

